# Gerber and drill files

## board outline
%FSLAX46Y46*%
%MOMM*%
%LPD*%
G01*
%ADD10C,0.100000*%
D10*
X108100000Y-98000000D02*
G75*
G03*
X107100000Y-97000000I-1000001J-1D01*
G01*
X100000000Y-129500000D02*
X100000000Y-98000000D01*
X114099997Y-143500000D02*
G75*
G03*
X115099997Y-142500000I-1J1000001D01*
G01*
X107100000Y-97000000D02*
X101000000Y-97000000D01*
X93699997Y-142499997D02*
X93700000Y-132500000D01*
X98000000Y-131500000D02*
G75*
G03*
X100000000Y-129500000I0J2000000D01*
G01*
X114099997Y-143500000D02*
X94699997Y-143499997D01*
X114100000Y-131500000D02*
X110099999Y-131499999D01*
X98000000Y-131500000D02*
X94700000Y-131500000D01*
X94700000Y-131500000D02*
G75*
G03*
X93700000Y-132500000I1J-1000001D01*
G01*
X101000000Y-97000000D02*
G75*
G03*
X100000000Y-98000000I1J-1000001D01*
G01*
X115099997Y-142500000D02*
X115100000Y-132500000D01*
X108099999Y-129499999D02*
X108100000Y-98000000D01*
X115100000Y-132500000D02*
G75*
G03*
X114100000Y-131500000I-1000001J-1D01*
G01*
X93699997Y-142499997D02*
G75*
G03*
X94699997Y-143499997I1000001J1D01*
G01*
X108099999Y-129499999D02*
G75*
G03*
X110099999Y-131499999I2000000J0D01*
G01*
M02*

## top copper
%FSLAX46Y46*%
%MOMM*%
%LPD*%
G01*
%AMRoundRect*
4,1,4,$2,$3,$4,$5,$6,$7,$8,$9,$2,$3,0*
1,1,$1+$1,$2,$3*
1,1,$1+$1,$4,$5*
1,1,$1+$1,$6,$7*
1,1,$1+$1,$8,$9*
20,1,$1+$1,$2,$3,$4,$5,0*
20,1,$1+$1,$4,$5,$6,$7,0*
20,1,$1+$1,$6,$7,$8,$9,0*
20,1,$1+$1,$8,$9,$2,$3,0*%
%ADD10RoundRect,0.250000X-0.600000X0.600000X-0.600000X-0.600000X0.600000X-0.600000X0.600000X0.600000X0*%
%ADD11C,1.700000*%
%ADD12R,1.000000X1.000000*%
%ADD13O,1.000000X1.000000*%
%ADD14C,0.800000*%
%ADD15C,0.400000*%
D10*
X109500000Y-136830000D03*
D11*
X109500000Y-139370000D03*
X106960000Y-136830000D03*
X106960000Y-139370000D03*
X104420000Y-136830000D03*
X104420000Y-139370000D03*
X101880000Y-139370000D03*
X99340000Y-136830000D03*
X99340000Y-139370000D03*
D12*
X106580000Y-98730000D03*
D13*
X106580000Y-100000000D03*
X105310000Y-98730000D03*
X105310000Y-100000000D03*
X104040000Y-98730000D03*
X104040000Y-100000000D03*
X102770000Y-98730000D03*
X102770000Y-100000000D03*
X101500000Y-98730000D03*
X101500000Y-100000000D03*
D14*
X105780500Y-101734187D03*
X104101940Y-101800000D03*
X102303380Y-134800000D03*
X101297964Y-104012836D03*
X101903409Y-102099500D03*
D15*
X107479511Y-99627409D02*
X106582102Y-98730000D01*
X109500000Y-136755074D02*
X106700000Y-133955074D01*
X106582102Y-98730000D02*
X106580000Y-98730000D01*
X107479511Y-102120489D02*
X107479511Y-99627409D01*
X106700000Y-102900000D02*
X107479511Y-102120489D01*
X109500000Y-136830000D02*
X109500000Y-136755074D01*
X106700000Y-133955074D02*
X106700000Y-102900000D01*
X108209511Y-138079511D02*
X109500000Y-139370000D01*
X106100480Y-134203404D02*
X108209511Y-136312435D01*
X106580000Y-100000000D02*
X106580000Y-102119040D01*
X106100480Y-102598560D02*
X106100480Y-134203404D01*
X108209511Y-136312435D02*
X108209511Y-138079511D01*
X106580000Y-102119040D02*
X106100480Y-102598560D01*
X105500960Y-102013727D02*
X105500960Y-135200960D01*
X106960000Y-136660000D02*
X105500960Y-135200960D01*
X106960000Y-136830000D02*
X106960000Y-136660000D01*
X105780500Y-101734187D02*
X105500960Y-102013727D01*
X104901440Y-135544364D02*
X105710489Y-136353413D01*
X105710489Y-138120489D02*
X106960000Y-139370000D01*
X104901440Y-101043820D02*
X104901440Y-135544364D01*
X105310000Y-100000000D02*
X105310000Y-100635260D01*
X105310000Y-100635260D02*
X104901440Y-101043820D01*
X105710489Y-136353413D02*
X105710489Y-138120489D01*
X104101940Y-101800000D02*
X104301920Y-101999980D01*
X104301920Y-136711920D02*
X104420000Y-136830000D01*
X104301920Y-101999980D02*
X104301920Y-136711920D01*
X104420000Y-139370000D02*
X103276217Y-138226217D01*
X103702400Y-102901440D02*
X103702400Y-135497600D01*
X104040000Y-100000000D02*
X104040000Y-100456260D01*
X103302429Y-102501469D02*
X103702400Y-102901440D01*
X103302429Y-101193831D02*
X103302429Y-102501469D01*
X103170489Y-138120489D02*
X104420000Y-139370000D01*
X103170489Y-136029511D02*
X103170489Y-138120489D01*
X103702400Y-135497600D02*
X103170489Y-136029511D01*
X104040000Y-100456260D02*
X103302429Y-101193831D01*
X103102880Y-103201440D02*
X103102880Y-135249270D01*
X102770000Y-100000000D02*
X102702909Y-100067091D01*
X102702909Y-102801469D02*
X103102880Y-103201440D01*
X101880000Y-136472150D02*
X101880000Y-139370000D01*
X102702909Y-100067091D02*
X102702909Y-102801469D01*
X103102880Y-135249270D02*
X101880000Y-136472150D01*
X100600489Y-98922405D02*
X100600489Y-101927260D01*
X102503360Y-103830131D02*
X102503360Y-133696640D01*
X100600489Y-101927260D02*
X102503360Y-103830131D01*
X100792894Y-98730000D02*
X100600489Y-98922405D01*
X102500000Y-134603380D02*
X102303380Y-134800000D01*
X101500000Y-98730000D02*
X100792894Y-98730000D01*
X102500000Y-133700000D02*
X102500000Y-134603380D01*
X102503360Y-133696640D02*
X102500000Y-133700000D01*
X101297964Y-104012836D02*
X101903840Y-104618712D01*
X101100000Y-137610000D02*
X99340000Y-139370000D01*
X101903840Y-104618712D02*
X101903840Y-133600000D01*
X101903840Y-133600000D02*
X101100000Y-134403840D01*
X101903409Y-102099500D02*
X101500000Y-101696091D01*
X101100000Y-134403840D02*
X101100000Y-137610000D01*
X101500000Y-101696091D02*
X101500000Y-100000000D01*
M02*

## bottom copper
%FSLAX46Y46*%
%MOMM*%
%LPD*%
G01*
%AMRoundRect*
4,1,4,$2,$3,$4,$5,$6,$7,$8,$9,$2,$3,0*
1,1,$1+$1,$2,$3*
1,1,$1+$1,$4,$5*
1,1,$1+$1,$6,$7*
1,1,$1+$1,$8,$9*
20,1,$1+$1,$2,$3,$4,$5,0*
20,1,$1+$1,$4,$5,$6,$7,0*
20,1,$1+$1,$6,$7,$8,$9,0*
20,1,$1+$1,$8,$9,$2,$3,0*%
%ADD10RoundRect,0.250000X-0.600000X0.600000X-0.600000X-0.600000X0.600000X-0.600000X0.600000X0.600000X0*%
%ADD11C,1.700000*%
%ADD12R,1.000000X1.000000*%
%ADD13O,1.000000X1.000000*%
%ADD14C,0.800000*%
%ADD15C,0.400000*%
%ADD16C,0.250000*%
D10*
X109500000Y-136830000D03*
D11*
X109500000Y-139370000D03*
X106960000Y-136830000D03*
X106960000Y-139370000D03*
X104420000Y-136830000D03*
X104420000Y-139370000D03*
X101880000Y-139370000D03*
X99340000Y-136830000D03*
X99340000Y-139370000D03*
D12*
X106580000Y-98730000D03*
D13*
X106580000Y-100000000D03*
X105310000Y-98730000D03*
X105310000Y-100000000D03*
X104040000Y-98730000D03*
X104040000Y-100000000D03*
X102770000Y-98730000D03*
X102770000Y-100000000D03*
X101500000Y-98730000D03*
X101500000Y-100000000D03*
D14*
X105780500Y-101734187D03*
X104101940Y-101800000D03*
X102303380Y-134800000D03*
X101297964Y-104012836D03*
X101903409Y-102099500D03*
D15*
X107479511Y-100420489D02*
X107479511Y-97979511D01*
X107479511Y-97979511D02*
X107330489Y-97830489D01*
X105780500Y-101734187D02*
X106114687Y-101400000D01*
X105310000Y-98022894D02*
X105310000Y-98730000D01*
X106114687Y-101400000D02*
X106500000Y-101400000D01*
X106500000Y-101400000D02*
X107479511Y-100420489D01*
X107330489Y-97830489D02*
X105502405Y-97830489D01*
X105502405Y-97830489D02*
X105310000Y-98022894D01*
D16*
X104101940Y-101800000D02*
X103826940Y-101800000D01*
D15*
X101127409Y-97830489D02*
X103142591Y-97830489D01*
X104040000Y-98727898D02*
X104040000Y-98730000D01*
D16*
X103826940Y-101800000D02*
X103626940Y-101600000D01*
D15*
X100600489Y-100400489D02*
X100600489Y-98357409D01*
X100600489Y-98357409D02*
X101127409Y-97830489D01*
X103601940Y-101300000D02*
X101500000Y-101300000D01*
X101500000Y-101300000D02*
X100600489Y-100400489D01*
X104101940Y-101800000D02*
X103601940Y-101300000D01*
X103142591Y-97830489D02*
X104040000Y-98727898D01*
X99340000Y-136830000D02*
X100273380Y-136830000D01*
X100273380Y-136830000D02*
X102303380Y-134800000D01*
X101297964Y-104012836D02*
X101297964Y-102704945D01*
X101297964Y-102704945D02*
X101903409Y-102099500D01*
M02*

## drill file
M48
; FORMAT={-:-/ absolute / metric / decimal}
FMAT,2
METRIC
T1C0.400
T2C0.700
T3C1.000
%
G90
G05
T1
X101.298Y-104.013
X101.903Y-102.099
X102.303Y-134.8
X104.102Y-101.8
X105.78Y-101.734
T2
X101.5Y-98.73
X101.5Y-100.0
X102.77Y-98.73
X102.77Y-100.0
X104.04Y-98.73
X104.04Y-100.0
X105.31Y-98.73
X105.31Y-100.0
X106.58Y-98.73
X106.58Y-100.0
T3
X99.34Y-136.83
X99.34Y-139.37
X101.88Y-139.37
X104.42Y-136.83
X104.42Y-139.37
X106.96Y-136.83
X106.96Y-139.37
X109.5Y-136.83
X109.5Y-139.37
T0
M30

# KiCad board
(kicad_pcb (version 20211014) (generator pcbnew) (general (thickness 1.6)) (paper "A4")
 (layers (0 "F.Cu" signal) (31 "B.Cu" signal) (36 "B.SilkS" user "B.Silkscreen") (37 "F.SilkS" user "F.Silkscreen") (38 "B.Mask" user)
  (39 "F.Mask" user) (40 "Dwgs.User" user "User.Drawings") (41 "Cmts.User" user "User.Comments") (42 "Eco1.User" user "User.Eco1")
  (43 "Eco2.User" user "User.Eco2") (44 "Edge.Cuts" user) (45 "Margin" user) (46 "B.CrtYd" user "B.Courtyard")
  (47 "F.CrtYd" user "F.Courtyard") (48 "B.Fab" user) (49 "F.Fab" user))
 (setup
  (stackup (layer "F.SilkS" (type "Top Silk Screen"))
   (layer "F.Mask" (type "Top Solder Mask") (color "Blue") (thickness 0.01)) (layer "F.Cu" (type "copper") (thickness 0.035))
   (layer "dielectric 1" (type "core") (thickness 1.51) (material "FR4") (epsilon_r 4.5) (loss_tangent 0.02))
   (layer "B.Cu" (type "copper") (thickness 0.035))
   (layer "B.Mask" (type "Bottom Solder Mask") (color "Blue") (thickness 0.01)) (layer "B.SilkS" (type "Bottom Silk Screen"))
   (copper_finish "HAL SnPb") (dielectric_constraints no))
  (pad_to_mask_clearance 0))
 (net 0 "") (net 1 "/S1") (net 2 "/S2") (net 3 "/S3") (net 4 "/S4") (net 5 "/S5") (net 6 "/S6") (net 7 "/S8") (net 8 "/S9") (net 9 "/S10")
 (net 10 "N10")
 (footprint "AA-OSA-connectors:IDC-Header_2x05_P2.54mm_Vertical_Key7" (layer "F.Cu") (at 109.5 136.83 -90)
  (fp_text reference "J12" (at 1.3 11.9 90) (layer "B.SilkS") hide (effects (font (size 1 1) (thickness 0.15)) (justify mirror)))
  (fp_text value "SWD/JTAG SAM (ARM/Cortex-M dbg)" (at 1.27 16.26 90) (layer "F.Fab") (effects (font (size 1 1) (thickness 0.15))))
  (pad "1" thru_hole roundrect (at 0 0 270) (size 1.7 1.7) (drill 1) (layers *.Cu *.Mask) (roundrect_rratio 0.1470588235) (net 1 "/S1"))
  (pad "2" thru_hole circle (at 2.54 0 270) (size 1.7 1.7) (drill 1) (layers *.Cu *.Mask) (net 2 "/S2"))
  (pad "3" thru_hole circle (at 0 2.54 270) (size 1.7 1.7) (drill 1) (layers *.Cu *.Mask) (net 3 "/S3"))
  (pad "4" thru_hole circle (at 2.54 2.54 270) (size 1.7 1.7) (drill 1) (layers *.Cu *.Mask) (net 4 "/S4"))
  (pad "5" thru_hole circle (at 0 5.08 270) (size 1.7 1.7) (drill 1) (layers *.Cu *.Mask) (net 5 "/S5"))
  (pad "6" thru_hole circle (at 2.54 5.08 270) (size 1.7 1.7) (drill 1) (layers *.Cu *.Mask) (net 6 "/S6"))
  (pad "8" thru_hole circle (at 2.54 7.62 270) (size 1.7 1.7) (drill 1) (layers *.Cu *.Mask) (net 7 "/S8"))
  (pad "9" thru_hole circle (at 0 10.16 270) (size 1.7 1.7) (drill 1) (layers *.Cu *.Mask) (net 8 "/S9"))
  (pad "10" thru_hole circle (at 2.54 10.16 270) (size 1.7 1.7) (drill 1) (layers *.Cu *.Mask) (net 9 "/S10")))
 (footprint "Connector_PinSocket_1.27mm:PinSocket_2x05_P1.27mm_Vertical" (layer "B.Cu") (at 106.58 98.73 90)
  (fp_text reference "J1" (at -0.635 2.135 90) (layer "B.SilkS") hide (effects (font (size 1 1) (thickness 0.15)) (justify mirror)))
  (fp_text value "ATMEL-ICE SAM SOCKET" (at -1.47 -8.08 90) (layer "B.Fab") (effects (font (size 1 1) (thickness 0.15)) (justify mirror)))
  (pad "1" thru_hole rect locked (at 0 0 90) (size 1 1) (drill 0.7) (layers *.Cu *.Mask) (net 1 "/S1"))
  (pad "2" thru_hole oval locked (at -1.27 0 90) (size 1 1) (drill 0.7) (layers *.Cu *.Mask) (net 2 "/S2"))
  (pad "3" thru_hole oval locked (at 0 -1.27 90) (size 1 1) (drill 0.7) (layers *.Cu *.Mask) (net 3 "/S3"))
  (pad "4" thru_hole oval locked (at -1.27 -1.27 90) (size 1 1) (drill 0.7) (layers *.Cu *.Mask) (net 4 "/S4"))
  (pad "5" thru_hole oval locked (at 0 -2.54 90) (size 1 1) (drill 0.7) (layers *.Cu *.Mask) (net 5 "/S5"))
  (pad "6" thru_hole oval locked (at -1.27 -2.54 90) (size 1 1) (drill 0.7) (layers *.Cu *.Mask) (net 6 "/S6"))
  (pad "7" thru_hole oval locked (at 0 -3.81 90) (size 1 1) (drill 0.7) (layers *.Cu *.Mask) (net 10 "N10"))
  (pad "8" thru_hole oval locked (at -1.27 -3.81 90) (size 1 1) (drill 0.7) (layers *.Cu *.Mask) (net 7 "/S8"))
  (pad "9" thru_hole oval locked (at 0 -5.08 90) (size 1 1) (drill 0.7) (layers *.Cu *.Mask) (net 8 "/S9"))
  (pad "10" thru_hole oval locked (at -1.27 -5.08 90) (size 1 1) (drill 0.7) (layers *.Cu *.Mask) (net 9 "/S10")))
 (gr_arc (start 107.1 97) (mid 107.807106 97.292894) (end 108.1 98) (layer "Edge.Cuts") (width 0.1))
 (gr_line (start 100 129.5) (end 100 98) (layer "Edge.Cuts") (width 0.1))
 (gr_arc (start 115.099997 142.5) (mid 114.807103 143.207106) (end 114.099997 143.5) (layer "Edge.Cuts") (width 0.1))
 (gr_line (start 107.1 97) (end 101 97) (layer "Edge.Cuts") (width 0.1))
 (gr_line (start 93.699997 142.499997) (end 93.7 132.5) (layer "Edge.Cuts") (width 0.1))
 (gr_arc (start 100 129.5) (mid 99.414214 130.914214) (end 98 131.5) (layer "Edge.Cuts") (width 0.1))
 (gr_line (start 114.099997 143.5) (end 94.699997 143.499997) (layer "Edge.Cuts") (width 0.1))
 (gr_line (start 114.1 131.5) (end 110.099999 131.499999) (layer "Edge.Cuts") (width 0.1))
 (gr_arc (start 93.7 132.5) (mid 93.992894 131.792894) (end 94.7 131.5) (layer "Edge.Cuts") (width 0.1))
 (gr_arc (start 100 98) (mid 100.292894 97.292894) (end 101 97) (layer "Edge.Cuts") (width 0.1))
 (gr_line (start 115.099997 142.5) (end 115.1 132.5) (layer "Edge.Cuts") (width 0.1))
 (gr_line (start 98 131.5) (end 94.7 131.5) (layer "Edge.Cuts") (width 0.1))
 (gr_line (start 108.099999 129.499999) (end 108.1 98) (layer "Edge.Cuts") (width 0.1))
 (gr_arc (start 114.1 131.5) (mid 114.807106 131.792894) (end 115.1 132.5) (layer "Edge.Cuts") (width 0.1))
 (gr_arc (start 94.699997 143.499997) (mid 93.992891 143.207103) (end 93.699997 142.499997) (layer "Edge.Cuts") (width 0.1))
 (gr_arc (start 110.099999 131.499999) (mid 108.685785 130.914213) (end 108.099999 129.499999) (layer "Edge.Cuts") (width 0.1))
 (segment (start 107.479511 99.627409) (end 106.582102 98.73) (width 0.4) (layer "F.Cu") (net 1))
 (segment (start 109.5 136.755074) (end 106.7 133.955074) (width 0.4) (layer "F.Cu") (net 1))
 (segment (start 106.582102 98.73) (end 106.58 98.73) (width 0.4) (layer "F.Cu") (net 1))
 (segment (start 107.479511 102.120489) (end 107.479511 99.627409) (width 0.4) (layer "F.Cu") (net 1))
 (segment (start 106.7 102.9) (end 107.479511 102.120489) (width 0.4) (layer "F.Cu") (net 1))
 (segment (start 109.5 136.83) (end 109.5 136.755074) (width 0.4) (layer "F.Cu") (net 1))
 (segment (start 106.7 133.955074) (end 106.7 102.9) (width 0.4) (layer "F.Cu") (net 1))
 (segment (start 108.209511 138.079511) (end 109.5 139.37) (width 0.4) (layer "F.Cu") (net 2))
 (segment (start 106.10048 134.203404) (end 108.209511 136.312435) (width 0.4) (layer "F.Cu") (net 2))
 (segment (start 106.58 100) (end 106.58 102.11904) (width 0.4) (layer "F.Cu") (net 2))
 (segment (start 106.10048 102.59856) (end 106.10048 134.203404) (width 0.4) (layer "F.Cu") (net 2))
 (segment (start 108.209511 136.312435) (end 108.209511 138.079511) (width 0.4) (layer "F.Cu") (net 2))
 (segment (start 106.58 102.11904) (end 106.10048 102.59856) (width 0.4) (layer "F.Cu") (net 2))
 (segment (start 105.50096 102.013727) (end 105.50096 135.20096) (width 0.4) (layer "F.Cu") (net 3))
 (segment (start 106.96 136.66) (end 105.50096 135.20096) (width 0.4) (layer "F.Cu") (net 3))
 (segment (start 106.96 136.83) (end 106.96 136.66) (width 0.4) (layer "F.Cu") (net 3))
 (segment (start 105.7805 101.734187) (end 105.50096 102.013727) (width 0.4) (layer "F.Cu") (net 3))
 (via (at 105.7805 101.734187) (size 0.8) (drill 0.4) (layers "F.Cu" "B.Cu") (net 3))
 (segment (start 107.479511 100.420489) (end 107.479511 97.979511) (width 0.4) (layer "B.Cu") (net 3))
 (segment (start 107.479511 97.979511) (end 107.330489 97.830489) (width 0.4) (layer "B.Cu") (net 3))
 (segment (start 105.7805 101.734187) (end 106.114687 101.4) (width 0.4) (layer "B.Cu") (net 3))
 (segment (start 105.31 98.022894) (end 105.31 98.73) (width 0.4) (layer "B.Cu") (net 3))
 (segment (start 106.114687 101.4) (end 106.5 101.4) (width 0.4) (layer "B.Cu") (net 3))
 (segment (start 106.5 101.4) (end 107.479511 100.420489) (width 0.4) (layer "B.Cu") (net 3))
 (segment (start 107.330489 97.830489) (end 105.502405 97.830489) (width 0.4) (layer "B.Cu") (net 3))
 (segment (start 105.502405 97.830489) (end 105.31 98.022894) (width 0.4) (layer "B.Cu") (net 3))
 (segment (start 104.90144 135.544364) (end 105.710489 136.353413) (width 0.4) (layer "F.Cu") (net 4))
 (segment (start 105.710489 138.120489) (end 106.96 139.37) (width 0.4) (layer "F.Cu") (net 4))
 (segment (start 104.90144 101.04382) (end 104.90144 135.544364) (width 0.4) (layer "F.Cu") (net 4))
 (segment (start 105.31 100) (end 105.31 100.63526) (width 0.4) (layer "F.Cu") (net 4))
 (segment (start 105.31 100.63526) (end 104.90144 101.04382) (width 0.4) (layer "F.Cu") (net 4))
 (segment (start 105.710489 136.353413) (end 105.710489 138.120489) (width 0.4) (layer "F.Cu") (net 4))
 (segment (start 104.10194 101.8) (end 104.30192 101.99998) (width 0.4) (layer "F.Cu") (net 5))
 (segment (start 104.30192 136.71192) (end 104.42 136.83) (width 0.4) (layer "F.Cu") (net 5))
 (segment (start 104.30192 101.99998) (end 104.30192 136.71192) (width 0.4) (layer "F.Cu") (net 5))
 (via (at 104.10194 101.8) (size 0.8) (drill 0.4) (layers "F.Cu" "B.Cu") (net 5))
 (segment (start 104.10194 101.8) (end 103.82694 101.8) (width 0.25) (layer "B.Cu") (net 5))
 (segment (start 101.127409 97.830489) (end 103.142591 97.830489) (width 0.4) (layer "B.Cu") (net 5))
 (segment (start 104.04 98.727898) (end 104.04 98.73) (width 0.4) (layer "B.Cu") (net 5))
 (segment (start 103.82694 101.8) (end 103.62694 101.6) (width 0.25) (layer "B.Cu") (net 5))
 (segment (start 100.600489 100.400489) (end 100.600489 98.357409) (width 0.4) (layer "B.Cu") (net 5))
 (segment (start 100.600489 98.357409) (end 101.127409 97.830489) (width 0.4) (layer "B.Cu") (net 5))
 (segment (start 103.60194 101.3) (end 101.5 101.3) (width 0.4) (layer "B.Cu") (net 5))
 (segment (start 101.5 101.3) (end 100.600489 100.400489) (width 0.4) (layer "B.Cu") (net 5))
 (segment (start 104.10194 101.8) (end 103.60194 101.3) (width 0.4) (layer "B.Cu") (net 5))
 (segment (start 103.142591 97.830489) (end 104.04 98.727898) (width 0.4) (layer "B.Cu") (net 5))
 (segment (start 104.42 139.37) (end 103.276217 138.226217) (width 0.4) (layer "F.Cu") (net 6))
 (segment (start 103.7024 102.90144) (end 103.7024 135.4976) (width 0.4) (layer "F.Cu") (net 6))
 (segment (start 104.04 100) (end 104.04 100.45626) (width 0.4) (layer "F.Cu") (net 6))
 (segment (start 103.302429 102.501469) (end 103.7024 102.90144) (width 0.4) (layer "F.Cu") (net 6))
 (segment (start 103.302429 101.193831) (end 103.302429 102.501469) (width 0.4) (layer "F.Cu") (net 6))
 (segment (start 103.170489 138.120489) (end 104.42 139.37) (width 0.4) (layer "F.Cu") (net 6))
 (segment (start 103.170489 136.029511) (end 103.170489 138.120489) (width 0.4) (layer "F.Cu") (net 6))
 (segment (start 103.7024 135.4976) (end 103.170489 136.029511) (width 0.4) (layer "F.Cu") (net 6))
 (segment (start 104.04 100.45626) (end 103.302429 101.193831) (width 0.4) (layer "F.Cu") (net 6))
 (segment (start 103.10288 103.20144) (end 103.10288 135.24927) (width 0.4) (layer "F.Cu") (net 7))
 (segment (start 102.77 100) (end 102.702909 100.067091) (width 0.4) (layer "F.Cu") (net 7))
 (segment (start 102.702909 102.801469) (end 103.10288 103.20144) (width 0.4) (layer "F.Cu") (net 7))
 (segment (start 101.88 136.47215) (end 101.88 139.37) (width 0.4) (layer "F.Cu") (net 7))
 (segment (start 102.702909 100.067091) (end 102.702909 102.801469) (width 0.4) (layer "F.Cu") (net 7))
 (segment (start 103.10288 135.24927) (end 101.88 136.47215) (width 0.4) (layer "F.Cu") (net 7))
 (segment (start 100.600489 98.922405) (end 100.600489 101.92726) (width 0.4) (layer "F.Cu") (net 8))
 (segment (start 102.50336 103.830131) (end 102.50336 133.69664) (width 0.4) (layer "F.Cu") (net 8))
 (segment (start 100.600489 101.92726) (end 102.50336 103.830131) (width 0.4) (layer "F.Cu") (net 8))
 (segment (start 100.792894 98.73) (end 100.600489 98.922405) (width 0.4) (layer "F.Cu") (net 8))
 (segment (start 102.5 134.60338) (end 102.30338 134.8) (width 0.4) (layer "F.Cu") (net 8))
 (segment (start 101.5 98.73) (end 100.792894 98.73) (width 0.4) (layer "F.Cu") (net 8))
 (segment (start 102.5 133.7) (end 102.5 134.60338) (width 0.4) (layer "F.Cu") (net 8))
 (segment (start 102.50336 133.69664) (end 102.5 133.7) (width 0.4) (layer "F.Cu") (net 8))
 (via (at 102.30338 134.8) (size 0.8) (drill 0.4) (layers "F.Cu" "B.Cu") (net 8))
 (segment (start 99.34 136.83) (end 100.27338 136.83) (width 0.4) (layer "B.Cu") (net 8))
 (segment (start 100.27338 136.83) (end 102.30338 134.8) (width 0.4) (layer "B.Cu") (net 8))
 (segment (start 101.297964 104.012836) (end 101.90384 104.618712) (width 0.4) (layer "F.Cu") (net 9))
 (segment (start 101.1 137.61) (end 99.34 139.37) (width 0.4) (layer "F.Cu") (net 9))
 (segment (start 101.90384 104.618712) (end 101.90384 133.6) (width 0.4) (layer "F.Cu") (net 9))
 (segment (start 101.90384 133.6) (end 101.1 134.40384) (width 0.4) (layer "F.Cu") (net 9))
 (segment (start 101.903409 102.0995) (end 101.5 101.696091) (width 0.4) (layer "F.Cu") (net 9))
 (segment (start 101.1 134.40384) (end 101.1 137.61) (width 0.4) (layer "F.Cu") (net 9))
 (segment (start 101.5 101.696091) (end 101.5 100) (width 0.4) (layer "F.Cu") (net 9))
 (via (at 101.297964 104.012836) (size 0.8) (drill 0.4) (layers "F.Cu" "B.Cu") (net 9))
 (via (at 101.903409 102.0995) (size 0.8) (drill 0.4) (layers "F.Cu" "B.Cu") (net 9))
 (segment (start 101.297964 104.012836) (end 101.297964 102.704945) (width 0.4) (layer "B.Cu") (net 9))
 (segment (start 101.297964 102.704945) (end 101.903409 102.0995) (width 0.4) (layer "B.Cu") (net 9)))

